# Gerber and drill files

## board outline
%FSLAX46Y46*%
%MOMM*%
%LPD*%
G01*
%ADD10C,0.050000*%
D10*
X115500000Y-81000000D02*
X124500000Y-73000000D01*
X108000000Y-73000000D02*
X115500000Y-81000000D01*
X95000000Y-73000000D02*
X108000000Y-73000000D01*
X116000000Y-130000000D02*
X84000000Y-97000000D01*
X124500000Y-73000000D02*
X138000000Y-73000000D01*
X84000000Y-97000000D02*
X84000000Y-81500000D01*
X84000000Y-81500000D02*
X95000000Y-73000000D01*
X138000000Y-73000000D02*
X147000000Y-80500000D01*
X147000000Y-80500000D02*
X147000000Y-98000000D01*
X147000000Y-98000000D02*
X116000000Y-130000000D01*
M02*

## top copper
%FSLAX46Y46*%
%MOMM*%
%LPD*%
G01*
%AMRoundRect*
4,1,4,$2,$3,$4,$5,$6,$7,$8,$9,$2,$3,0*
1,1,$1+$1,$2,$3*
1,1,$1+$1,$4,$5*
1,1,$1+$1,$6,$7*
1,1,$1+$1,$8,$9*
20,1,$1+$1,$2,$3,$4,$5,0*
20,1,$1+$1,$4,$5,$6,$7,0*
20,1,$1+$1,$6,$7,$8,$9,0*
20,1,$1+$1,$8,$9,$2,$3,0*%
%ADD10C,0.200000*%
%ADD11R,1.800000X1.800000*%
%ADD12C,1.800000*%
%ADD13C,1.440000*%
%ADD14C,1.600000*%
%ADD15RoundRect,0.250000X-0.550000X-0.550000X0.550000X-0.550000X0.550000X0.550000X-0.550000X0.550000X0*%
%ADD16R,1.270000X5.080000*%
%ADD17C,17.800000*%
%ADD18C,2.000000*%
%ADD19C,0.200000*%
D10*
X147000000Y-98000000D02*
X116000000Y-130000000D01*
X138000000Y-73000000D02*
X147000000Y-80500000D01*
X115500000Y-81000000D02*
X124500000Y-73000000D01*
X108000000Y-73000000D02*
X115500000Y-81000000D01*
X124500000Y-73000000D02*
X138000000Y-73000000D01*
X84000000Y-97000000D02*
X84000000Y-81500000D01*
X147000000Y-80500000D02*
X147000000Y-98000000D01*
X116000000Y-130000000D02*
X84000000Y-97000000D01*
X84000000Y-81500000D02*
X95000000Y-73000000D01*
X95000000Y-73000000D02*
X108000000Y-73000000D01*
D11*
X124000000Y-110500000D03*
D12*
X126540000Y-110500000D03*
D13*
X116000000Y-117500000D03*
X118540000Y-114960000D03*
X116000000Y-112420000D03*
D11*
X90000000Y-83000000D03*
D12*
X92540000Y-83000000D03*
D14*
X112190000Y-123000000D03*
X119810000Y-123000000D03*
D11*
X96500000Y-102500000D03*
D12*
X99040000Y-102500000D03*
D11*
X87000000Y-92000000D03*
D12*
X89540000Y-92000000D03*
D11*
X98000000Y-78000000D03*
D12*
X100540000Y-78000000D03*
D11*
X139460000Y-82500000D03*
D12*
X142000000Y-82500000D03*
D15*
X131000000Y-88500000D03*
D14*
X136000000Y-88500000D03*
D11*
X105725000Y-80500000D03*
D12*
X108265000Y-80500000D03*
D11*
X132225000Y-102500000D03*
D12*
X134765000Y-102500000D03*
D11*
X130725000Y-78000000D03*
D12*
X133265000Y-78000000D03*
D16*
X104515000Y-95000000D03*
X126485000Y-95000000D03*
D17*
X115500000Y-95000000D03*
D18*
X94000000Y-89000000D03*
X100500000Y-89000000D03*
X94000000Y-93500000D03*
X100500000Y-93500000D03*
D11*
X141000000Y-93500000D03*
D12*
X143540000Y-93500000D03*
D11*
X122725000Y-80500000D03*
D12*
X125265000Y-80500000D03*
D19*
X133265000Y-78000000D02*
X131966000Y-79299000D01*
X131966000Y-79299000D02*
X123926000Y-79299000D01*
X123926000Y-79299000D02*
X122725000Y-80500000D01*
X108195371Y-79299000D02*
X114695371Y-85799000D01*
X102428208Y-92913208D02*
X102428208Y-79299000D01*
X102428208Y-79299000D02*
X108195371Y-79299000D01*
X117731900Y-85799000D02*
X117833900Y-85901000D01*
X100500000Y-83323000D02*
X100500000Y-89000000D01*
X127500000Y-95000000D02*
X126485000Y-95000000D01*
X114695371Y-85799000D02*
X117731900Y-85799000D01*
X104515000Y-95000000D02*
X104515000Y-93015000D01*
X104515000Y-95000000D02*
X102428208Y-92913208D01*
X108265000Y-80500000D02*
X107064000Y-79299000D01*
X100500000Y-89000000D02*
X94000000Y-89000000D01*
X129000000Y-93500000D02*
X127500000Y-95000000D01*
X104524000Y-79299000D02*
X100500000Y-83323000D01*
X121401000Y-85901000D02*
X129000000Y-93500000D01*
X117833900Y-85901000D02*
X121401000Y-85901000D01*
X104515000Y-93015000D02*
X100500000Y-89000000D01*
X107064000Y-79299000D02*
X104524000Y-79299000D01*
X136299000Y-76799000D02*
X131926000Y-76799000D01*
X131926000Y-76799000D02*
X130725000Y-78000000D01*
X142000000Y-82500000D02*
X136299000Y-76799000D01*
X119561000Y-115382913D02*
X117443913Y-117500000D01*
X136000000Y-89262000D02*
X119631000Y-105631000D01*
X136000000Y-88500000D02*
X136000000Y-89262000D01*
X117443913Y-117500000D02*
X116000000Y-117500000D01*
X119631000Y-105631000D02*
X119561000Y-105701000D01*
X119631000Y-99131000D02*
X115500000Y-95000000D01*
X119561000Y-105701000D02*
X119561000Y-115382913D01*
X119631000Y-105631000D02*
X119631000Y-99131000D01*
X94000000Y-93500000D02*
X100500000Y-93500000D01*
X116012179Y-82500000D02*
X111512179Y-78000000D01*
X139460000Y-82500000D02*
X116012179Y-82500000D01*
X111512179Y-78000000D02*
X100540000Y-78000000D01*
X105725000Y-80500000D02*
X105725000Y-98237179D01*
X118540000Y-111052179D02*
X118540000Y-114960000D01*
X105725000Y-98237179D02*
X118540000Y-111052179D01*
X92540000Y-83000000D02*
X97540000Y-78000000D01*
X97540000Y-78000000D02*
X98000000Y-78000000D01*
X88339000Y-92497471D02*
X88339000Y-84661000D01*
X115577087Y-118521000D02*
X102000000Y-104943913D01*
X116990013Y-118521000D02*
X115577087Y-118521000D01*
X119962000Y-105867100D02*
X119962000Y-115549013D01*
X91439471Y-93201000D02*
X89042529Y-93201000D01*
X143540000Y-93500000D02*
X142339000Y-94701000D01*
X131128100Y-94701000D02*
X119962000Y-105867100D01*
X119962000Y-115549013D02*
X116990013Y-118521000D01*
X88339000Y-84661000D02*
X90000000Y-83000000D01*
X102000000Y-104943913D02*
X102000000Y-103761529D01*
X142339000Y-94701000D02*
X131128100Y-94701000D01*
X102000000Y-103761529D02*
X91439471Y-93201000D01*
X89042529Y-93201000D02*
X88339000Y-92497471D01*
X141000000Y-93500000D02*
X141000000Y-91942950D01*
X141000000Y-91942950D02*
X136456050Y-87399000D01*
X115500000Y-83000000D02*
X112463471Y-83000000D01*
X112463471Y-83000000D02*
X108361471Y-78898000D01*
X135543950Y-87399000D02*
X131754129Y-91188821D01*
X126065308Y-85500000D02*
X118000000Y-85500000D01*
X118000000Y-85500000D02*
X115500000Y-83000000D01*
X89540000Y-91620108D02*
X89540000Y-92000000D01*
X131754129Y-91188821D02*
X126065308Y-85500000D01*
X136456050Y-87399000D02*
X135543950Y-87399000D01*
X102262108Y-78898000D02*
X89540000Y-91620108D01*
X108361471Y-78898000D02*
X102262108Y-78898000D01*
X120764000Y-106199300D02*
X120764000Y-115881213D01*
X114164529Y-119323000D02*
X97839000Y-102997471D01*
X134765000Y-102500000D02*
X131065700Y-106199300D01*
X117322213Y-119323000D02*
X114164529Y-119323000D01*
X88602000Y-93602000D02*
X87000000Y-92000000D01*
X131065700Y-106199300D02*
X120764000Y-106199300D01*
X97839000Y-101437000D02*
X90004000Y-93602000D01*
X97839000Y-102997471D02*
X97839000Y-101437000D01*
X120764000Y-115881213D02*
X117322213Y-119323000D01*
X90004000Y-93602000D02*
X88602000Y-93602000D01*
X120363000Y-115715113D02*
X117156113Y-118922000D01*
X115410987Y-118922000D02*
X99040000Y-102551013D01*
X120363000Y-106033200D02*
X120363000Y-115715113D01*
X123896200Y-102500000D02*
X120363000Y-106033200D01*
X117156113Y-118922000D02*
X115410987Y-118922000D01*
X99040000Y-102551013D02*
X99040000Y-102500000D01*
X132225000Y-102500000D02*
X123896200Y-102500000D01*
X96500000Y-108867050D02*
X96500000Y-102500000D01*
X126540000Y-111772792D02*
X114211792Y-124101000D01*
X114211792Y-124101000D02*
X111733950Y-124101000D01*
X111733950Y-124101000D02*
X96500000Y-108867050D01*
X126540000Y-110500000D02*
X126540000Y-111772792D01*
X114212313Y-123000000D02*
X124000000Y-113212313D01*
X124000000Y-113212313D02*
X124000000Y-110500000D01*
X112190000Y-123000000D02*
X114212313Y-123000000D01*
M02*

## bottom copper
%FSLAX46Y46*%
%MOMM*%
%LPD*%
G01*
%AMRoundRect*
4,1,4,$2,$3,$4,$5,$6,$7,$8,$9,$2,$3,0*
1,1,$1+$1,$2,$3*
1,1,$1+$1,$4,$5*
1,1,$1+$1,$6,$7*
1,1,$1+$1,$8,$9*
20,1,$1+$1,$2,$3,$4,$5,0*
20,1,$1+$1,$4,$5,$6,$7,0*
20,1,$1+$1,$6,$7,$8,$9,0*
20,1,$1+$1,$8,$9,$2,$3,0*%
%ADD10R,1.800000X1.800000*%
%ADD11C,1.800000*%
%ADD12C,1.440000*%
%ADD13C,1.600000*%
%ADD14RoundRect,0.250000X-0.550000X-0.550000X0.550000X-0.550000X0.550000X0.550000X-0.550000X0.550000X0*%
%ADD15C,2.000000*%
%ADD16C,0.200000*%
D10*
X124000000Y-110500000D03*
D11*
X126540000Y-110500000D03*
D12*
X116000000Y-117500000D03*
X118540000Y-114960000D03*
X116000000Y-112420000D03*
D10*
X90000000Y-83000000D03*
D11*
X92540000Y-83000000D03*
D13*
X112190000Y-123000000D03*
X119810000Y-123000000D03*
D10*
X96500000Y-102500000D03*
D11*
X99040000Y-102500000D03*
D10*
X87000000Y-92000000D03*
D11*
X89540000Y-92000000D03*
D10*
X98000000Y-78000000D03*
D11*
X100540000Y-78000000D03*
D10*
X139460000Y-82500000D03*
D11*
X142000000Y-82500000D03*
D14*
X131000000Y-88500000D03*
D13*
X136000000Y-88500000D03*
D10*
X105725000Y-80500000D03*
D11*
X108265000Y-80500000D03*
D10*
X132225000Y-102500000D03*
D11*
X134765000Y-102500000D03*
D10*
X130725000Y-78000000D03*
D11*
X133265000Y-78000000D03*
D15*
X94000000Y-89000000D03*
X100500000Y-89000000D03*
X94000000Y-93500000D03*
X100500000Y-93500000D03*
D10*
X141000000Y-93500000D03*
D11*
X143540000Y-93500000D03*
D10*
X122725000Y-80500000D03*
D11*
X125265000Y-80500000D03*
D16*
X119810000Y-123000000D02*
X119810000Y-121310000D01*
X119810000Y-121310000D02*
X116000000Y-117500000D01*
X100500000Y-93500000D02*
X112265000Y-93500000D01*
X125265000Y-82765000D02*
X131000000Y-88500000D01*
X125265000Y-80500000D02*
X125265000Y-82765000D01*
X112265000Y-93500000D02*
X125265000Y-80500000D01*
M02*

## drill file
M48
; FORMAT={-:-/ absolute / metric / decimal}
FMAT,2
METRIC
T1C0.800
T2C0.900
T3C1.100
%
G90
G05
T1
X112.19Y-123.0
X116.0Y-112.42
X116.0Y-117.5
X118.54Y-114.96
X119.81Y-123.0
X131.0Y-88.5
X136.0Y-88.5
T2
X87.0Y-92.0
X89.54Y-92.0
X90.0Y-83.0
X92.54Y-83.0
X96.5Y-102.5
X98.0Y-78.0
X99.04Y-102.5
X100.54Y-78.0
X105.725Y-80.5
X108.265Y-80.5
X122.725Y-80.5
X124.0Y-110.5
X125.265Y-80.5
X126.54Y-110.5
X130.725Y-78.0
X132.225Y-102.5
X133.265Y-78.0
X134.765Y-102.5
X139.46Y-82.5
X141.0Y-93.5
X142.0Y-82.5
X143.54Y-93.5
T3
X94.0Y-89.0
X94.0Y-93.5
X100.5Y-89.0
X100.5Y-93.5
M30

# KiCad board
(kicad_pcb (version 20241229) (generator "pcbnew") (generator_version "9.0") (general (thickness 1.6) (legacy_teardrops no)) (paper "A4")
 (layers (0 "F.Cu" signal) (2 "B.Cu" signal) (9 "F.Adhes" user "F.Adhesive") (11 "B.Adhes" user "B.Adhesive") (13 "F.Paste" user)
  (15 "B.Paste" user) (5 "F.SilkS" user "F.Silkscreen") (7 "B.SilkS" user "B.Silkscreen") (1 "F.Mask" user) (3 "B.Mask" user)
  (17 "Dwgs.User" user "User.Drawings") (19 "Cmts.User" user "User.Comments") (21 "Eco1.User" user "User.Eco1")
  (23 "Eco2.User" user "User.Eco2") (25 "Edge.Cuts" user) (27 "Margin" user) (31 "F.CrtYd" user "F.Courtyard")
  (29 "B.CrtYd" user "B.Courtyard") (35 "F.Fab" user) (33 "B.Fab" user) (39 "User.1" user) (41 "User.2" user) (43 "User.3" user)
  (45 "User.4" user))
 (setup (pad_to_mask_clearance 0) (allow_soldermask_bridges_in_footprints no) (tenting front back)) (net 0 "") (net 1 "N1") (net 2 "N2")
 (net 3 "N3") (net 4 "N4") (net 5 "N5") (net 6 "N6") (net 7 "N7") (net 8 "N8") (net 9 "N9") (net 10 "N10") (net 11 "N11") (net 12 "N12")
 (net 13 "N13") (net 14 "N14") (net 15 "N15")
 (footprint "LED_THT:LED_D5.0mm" (layer "F.Cu") (at 124 110.5)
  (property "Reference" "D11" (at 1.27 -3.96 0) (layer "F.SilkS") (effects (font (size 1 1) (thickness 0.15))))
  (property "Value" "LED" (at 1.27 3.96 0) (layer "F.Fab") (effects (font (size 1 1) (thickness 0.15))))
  (pad "1" thru_hole rect (at 0 0) (size 1.8 1.8) (drill 0.9) (layers "*.Cu" "*.Mask") (remove_unused_layers no) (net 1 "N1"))
  (pad "2" thru_hole circle (at 2.54 0) (size 1.8 1.8) (drill 0.9) (layers "*.Cu" "*.Mask") (remove_unused_layers no) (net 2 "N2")))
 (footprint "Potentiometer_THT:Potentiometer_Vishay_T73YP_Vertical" (layer "F.Cu") (at 116 117.5)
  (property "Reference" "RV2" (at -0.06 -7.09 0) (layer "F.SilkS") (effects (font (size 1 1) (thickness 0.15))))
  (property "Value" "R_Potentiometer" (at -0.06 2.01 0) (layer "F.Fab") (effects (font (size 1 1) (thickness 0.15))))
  (pad "1" thru_hole circle (at 0 0) (size 1.44 1.44) (drill 0.8) (layers "*.Cu" "*.Mask") (remove_unused_layers no) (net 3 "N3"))
  (pad "2" thru_hole circle (at 2.54 -2.54) (size 1.44 1.44) (drill 0.8) (layers "*.Cu" "*.Mask") (remove_unused_layers no) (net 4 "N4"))
  (pad "3" thru_hole circle (at 0 -5.08) (size 1.44 1.44) (drill 0.8) (layers "*.Cu" "*.Mask") (remove_unused_layers no) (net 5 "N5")))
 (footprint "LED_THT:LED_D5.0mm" (layer "F.Cu") (at 90 83)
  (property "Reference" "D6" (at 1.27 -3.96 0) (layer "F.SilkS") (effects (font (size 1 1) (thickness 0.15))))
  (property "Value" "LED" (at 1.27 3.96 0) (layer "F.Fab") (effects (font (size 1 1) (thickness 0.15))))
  (pad "1" thru_hole rect (at 0 0) (size 1.8 1.8) (drill 0.9) (layers "*.Cu" "*.Mask") (remove_unused_layers no) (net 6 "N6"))
  (pad "2" thru_hole circle (at 2.54 0) (size 1.8 1.8) (drill 0.9) (layers "*.Cu" "*.Mask") (remove_unused_layers no) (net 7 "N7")))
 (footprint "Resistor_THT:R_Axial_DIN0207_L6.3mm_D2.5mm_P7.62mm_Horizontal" (layer "F.Cu") (at 112.19 123)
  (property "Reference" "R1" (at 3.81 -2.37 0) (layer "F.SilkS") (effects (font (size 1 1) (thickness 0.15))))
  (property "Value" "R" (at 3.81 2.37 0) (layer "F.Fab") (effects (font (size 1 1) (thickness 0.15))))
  (pad "1" thru_hole circle (at 0 0) (size 1.6 1.6) (drill 0.8) (layers "*.Cu" "*.Mask") (remove_unused_layers no) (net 1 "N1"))
  (pad "2" thru_hole circle (at 7.62 0) (size 1.6 1.6) (drill 0.8) (layers "*.Cu" "*.Mask") (remove_unused_layers no) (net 3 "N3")))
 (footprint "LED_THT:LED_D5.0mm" (layer "F.Cu") (at 96.5 102.5)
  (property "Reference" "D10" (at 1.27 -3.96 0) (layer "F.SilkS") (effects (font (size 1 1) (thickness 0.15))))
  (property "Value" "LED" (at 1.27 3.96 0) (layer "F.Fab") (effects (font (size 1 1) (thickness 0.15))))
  (pad "1" thru_hole rect (at 0 0) (size 1.8 1.8) (drill 0.9) (layers "*.Cu" "*.Mask") (remove_unused_layers no) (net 2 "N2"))
  (pad "2" thru_hole circle (at 2.54 0) (size 1.8 1.8) (drill 0.9) (layers "*.Cu" "*.Mask") (remove_unused_layers no) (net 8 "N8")))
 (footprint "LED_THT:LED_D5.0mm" (layer "F.Cu") (at 87 92)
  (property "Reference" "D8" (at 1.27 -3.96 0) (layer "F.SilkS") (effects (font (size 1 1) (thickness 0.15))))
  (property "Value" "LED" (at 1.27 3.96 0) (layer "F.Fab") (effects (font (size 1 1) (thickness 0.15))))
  (pad "1" thru_hole rect (at 0 0) (size 1.8 1.8) (drill 0.9) (layers "*.Cu" "*.Mask") (remove_unused_layers no) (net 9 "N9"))
  (pad "2" thru_hole circle (at 2.54 0) (size 1.8 1.8) (drill 0.9) (layers "*.Cu" "*.Mask") (remove_unused_layers no) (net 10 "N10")))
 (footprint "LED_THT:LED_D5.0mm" (layer "F.Cu") (at 98 78)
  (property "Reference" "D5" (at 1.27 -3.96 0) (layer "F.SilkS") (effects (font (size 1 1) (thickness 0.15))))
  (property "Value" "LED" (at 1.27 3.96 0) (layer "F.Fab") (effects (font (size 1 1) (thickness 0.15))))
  (pad "1" thru_hole rect (at 0 0) (size 1.8 1.8) (drill 0.9) (layers "*.Cu" "*.Mask") (remove_unused_layers no) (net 7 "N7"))
  (pad "2" thru_hole circle (at 2.54 0) (size 1.8 1.8) (drill 0.9) (layers "*.Cu" "*.Mask") (remove_unused_layers no) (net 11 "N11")))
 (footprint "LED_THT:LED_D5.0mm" (layer "F.Cu") (at 139.46 82.5)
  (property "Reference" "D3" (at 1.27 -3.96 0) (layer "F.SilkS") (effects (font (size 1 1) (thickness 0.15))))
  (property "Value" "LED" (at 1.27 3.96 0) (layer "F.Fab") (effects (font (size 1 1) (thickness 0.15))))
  (pad "1" thru_hole rect (at 0 0) (size 1.8 1.8) (drill 0.9) (layers "*.Cu" "*.Mask") (remove_unused_layers no) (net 11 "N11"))
  (pad "2" thru_hole circle (at 2.54 0) (size 1.8 1.8) (drill 0.9) (layers "*.Cu" "*.Mask") (remove_unused_layers no) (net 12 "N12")))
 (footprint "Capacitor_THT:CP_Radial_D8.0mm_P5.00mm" (layer "F.Cu") (at 131 88.5)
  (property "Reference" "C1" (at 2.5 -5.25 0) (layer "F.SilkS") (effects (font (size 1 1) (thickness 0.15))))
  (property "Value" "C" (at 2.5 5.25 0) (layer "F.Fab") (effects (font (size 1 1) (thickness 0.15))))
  (pad "1" thru_hole roundrect (at 0 0) (size 1.6 1.6) (drill 0.8) (layers "*.Cu" "*.Mask") (remove_unused_layers no)
   (roundrect_rratio 0.15625) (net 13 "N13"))
  (pad "2" thru_hole circle (at 5 0) (size 1.6 1.6) (drill 0.8) (layers "*.Cu" "*.Mask") (remove_unused_layers no) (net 3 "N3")))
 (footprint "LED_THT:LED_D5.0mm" (layer "F.Cu") (at 105.725 80.5)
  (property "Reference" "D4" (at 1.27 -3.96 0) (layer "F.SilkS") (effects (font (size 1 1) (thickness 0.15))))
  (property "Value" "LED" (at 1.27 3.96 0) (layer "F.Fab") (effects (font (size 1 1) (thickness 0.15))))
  (pad "1" thru_hole rect (at 0 0) (size 1.8 1.8) (drill 0.9) (layers "*.Cu" "*.Mask") (remove_unused_layers no) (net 4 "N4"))
  (pad "2" thru_hole circle (at 2.54 0) (size 1.8 1.8) (drill 0.9) (layers "*.Cu" "*.Mask") (remove_unused_layers no) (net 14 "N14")))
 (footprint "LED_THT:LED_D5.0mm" (layer "F.Cu") (at 132.225 102.5)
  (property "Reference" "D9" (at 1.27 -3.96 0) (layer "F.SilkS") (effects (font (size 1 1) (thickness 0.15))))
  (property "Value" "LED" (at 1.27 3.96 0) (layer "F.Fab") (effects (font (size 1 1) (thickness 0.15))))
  (pad "1" thru_hole rect (at 0 0) (size 1.8 1.8) (drill 0.9) (layers "*.Cu" "*.Mask") (remove_unused_layers no) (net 8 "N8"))
  (pad "2" thru_hole circle (at 2.54 0) (size 1.8 1.8) (drill 0.9) (layers "*.Cu" "*.Mask") (remove_unused_layers no) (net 9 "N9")))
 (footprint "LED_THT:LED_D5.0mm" (layer "F.Cu") (at 130.725 78)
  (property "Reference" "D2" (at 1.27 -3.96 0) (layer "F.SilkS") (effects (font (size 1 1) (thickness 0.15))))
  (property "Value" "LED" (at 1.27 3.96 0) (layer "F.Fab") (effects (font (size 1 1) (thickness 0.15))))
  (pad "1" thru_hole rect (at 0 0) (size 1.8 1.8) (drill 0.9) (layers "*.Cu" "*.Mask") (remove_unused_layers no) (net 12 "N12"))
  (pad "2" thru_hole circle (at 2.54 0) (size 1.8 1.8) (drill 0.9) (layers "*.Cu" "*.Mask") (remove_unused_layers no) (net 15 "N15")))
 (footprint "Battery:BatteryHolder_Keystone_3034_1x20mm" (layer "F.Cu") (at 115.5 95)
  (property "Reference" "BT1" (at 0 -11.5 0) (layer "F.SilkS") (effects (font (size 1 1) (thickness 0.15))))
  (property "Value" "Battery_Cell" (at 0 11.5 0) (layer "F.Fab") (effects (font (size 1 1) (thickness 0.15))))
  (pad "1" smd rect (at -10.985 0) (size 1.27 5.08) (layers "F.Cu" "F.Mask" "F.Paste") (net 14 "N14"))
  (pad "1" smd rect (at 10.985 0) (size 1.27 5.08) (layers "F.Cu" "F.Mask" "F.Paste") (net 14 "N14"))
  (pad "2" smd circle (at 0 0) (size 17.8 17.8) (layers "F.Cu" "F.Mask") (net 3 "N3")))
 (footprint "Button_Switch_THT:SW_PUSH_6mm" (layer "F.Cu") (at 94 89)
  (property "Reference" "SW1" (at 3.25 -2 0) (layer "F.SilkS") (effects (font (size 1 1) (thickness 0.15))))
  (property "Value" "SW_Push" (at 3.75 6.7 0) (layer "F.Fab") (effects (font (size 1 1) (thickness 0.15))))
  (pad "1" thru_hole circle (at 0 0 90) (size 2 2) (drill 1.1) (layers "*.Cu" "*.Mask") (remove_unused_layers no) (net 14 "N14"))
  (pad "1" thru_hole circle (at 6.5 0 90) (size 2 2) (drill 1.1) (layers "*.Cu" "*.Mask") (remove_unused_layers no) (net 14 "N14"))
  (pad "2" thru_hole circle (at 0 4.5 90) (size 2 2) (drill 1.1) (layers "*.Cu" "*.Mask") (remove_unused_layers no) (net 13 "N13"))
  (pad "2" thru_hole circle (at 6.5 4.5 90) (size 2 2) (drill 1.1) (layers "*.Cu" "*.Mask") (remove_unused_layers no) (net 13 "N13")))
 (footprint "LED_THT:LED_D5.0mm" (layer "F.Cu") (at 141 93.5)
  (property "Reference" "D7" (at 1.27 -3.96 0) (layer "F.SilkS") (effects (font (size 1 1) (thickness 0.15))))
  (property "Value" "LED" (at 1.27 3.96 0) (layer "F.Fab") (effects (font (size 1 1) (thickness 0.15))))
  (pad "1" thru_hole rect (at 0 0) (size 1.8 1.8) (drill 0.9) (layers "*.Cu" "*.Mask") (remove_unused_layers no) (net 10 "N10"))
  (pad "2" thru_hole circle (at 2.54 0) (size 1.8 1.8) (drill 0.9) (layers "*.Cu" "*.Mask") (remove_unused_layers no) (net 6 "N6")))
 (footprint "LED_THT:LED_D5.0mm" (layer "F.Cu") (at 122.725 80.5)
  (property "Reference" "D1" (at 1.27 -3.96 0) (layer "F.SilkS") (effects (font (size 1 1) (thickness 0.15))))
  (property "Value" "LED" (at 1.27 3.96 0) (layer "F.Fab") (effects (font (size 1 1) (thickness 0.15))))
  (pad "1" thru_hole rect (at 0 0) (size 1.8 1.8) (drill 0.9) (layers "*.Cu" "*.Mask") (remove_unused_layers no) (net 15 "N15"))
  (pad "2" thru_hole circle (at 2.54 0) (size 1.8 1.8) (drill 0.9) (layers "*.Cu" "*.Mask") (remove_unused_layers no) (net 13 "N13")))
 (gr_line (start 147 98) (end 116 130) (stroke (width 0.2) (type default)) (layer "F.Cu"))
 (gr_line (start 138 73) (end 147 80.5) (stroke (width 0.2) (type default)) (layer "F.Cu"))
 (gr_line (start 115.5 81) (end 124.5 73) (stroke (width 0.2) (type default)) (layer "F.Cu"))
 (gr_line (start 108 73) (end 115.5 81) (stroke (width 0.2) (type default)) (layer "F.Cu"))
 (gr_line (start 124.5 73) (end 138 73) (stroke (width 0.2) (type default)) (layer "F.Cu"))
 (gr_line (start 84 97) (end 84 81.5) (stroke (width 0.2) (type default)) (layer "F.Cu"))
 (gr_line (start 147 80.5) (end 147 98) (stroke (width 0.2) (type default)) (layer "F.Cu"))
 (gr_line (start 116 130) (end 84 97) (stroke (width 0.2) (type default)) (layer "F.Cu"))
 (gr_line (start 84 81.5) (end 95 73) (stroke (width 0.2) (type default)) (layer "F.Cu"))
 (gr_line (start 95 73) (end 108 73) (stroke (width 0.2) (type default)) (layer "F.Cu"))
 (gr_line (start 115.5 81) (end 124.5 73) (stroke (width 0.05) (type default)) (layer "Edge.Cuts"))
 (gr_line (start 108 73) (end 115.5 81) (stroke (width 0.05) (type default)) (layer "Edge.Cuts"))
 (gr_line (start 95 73) (end 108 73) (stroke (width 0.05) (type default)) (layer "Edge.Cuts"))
 (gr_line (start 116 130) (end 84 97) (stroke (width 0.05) (type default)) (layer "Edge.Cuts"))
 (gr_line (start 124.5 73) (end 138 73) (stroke (width 0.05) (type default)) (layer "Edge.Cuts"))
 (gr_line (start 84 97) (end 84 81.5) (stroke (width 0.05) (type default)) (layer "Edge.Cuts"))
 (gr_line (start 84 81.5) (end 95 73) (stroke (width 0.05) (type default)) (layer "Edge.Cuts"))
 (gr_line (start 138 73) (end 147 80.5) (stroke (width 0.05) (type default)) (layer "Edge.Cuts"))
 (gr_line (start 147 80.5) (end 147 98) (stroke (width 0.05) (type default)) (layer "Edge.Cuts"))
 (gr_line (start 147 98) (end 116 130) (stroke (width 0.05) (type default)) (layer "Edge.Cuts"))
 (segment (start 133.265 78) (end 131.966 79.299) (width 0.2) (layer "F.Cu") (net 15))
 (segment (start 131.966 79.299) (end 123.926 79.299) (width 0.2) (layer "F.Cu") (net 15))
 (segment (start 123.926 79.299) (end 122.725 80.5) (width 0.2) (layer "F.Cu") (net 15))
 (segment (start 108.195371 79.299) (end 114.695371 85.799) (width 0.2) (layer "F.Cu") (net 14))
 (segment (start 102.428208 92.913208) (end 102.428208 79.299) (width 0.2) (layer "F.Cu") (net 14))
 (segment (start 102.428208 79.299) (end 108.195371 79.299) (width 0.2) (layer "F.Cu") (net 14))
 (segment (start 117.7319 85.799) (end 117.8339 85.901) (width 0.2) (layer "F.Cu") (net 14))
 (segment (start 100.5 83.323) (end 100.5 89) (width 0.2) (layer "F.Cu") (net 14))
 (segment (start 127.5 95) (end 126.485 95) (width 0.2) (layer "F.Cu") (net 14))
 (segment (start 114.695371 85.799) (end 117.7319 85.799) (width 0.2) (layer "F.Cu") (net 14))
 (segment (start 104.515 95) (end 104.515 93.015) (width 0.2) (layer "F.Cu") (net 14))
 (segment (start 104.515 95) (end 102.428208 92.913208) (width 0.2) (layer "F.Cu") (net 14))
 (segment (start 108.265 80.5) (end 107.064 79.299) (width 0.2) (layer "F.Cu") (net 14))
 (segment (start 100.5 89) (end 94 89) (width 0.2) (layer "F.Cu") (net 14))
 (segment (start 129 93.5) (end 127.5 95) (width 0.2) (layer "F.Cu") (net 14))
 (segment (start 104.524 79.299) (end 100.5 83.323) (width 0.2) (layer "F.Cu") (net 14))
 (segment (start 121.401 85.901) (end 129 93.5) (width 0.2) (layer "F.Cu") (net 14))
 (segment (start 117.8339 85.901) (end 121.401 85.901) (width 0.2) (layer "F.Cu") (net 14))
 (segment (start 104.515 93.015) (end 100.5 89) (width 0.2) (layer "F.Cu") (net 14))
 (segment (start 107.064 79.299) (end 104.524 79.299) (width 0.2) (layer "F.Cu") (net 14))
 (segment (start 136.299 76.799) (end 131.926 76.799) (width 0.2) (layer "F.Cu") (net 12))
 (segment (start 131.926 76.799) (end 130.725 78) (width 0.2) (layer "F.Cu") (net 12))
 (segment (start 142 82.5) (end 136.299 76.799) (width 0.2) (layer "F.Cu") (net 12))
 (segment (start 119.561 115.382913) (end 117.443913 117.5) (width 0.2) (layer "F.Cu") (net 3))
 (segment (start 136 89.262) (end 119.631 105.631) (width 0.2) (layer "F.Cu") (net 3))
 (segment (start 136 88.5) (end 136 89.262) (width 0.2) (layer "F.Cu") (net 3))
 (segment (start 117.443913 117.5) (end 116 117.5) (width 0.2) (layer "F.Cu") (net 3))
 (segment (start 119.631 105.631) (end 119.561 105.701) (width 0.2) (layer "F.Cu") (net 3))
 (segment (start 119.631 99.131) (end 115.5 95) (width 0.2) (layer "F.Cu") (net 3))
 (segment (start 119.561 105.701) (end 119.561 115.382913) (width 0.2) (layer "F.Cu") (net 3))
 (segment (start 119.631 105.631) (end 119.631 99.131) (width 0.2) (layer "F.Cu") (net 3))
 (segment (start 119.81 123) (end 119.81 121.31) (width 0.2) (layer "B.Cu") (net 3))
 (segment (start 119.81 121.31) (end 116 117.5) (width 0.2) (layer "B.Cu") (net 3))
 (segment (start 94 93.5) (end 100.5 93.5) (width 0.2) (layer "F.Cu") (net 13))
 (segment (start 100.5 93.5) (end 112.265 93.5) (width 0.2) (layer "B.Cu") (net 13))
 (segment (start 125.265 82.765) (end 131 88.5) (width 0.2) (layer "B.Cu") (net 13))
 (segment (start 125.265 80.5) (end 125.265 82.765) (width 0.2) (layer "B.Cu") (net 13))
 (segment (start 112.265 93.5) (end 125.265 80.5) (width 0.2) (layer "B.Cu") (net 13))
 (segment (start 116.012179 82.5) (end 111.512179 78) (width 0.2) (layer "F.Cu") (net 11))
 (segment (start 139.46 82.5) (end 116.012179 82.5) (width 0.2) (layer "F.Cu") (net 11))
 (segment (start 111.512179 78) (end 100.54 78) (width 0.2) (layer "F.Cu") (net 11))
 (segment (start 105.725 80.5) (end 105.725 98.237179) (width 0.2) (layer "F.Cu") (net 4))
 (segment (start 118.54 111.052179) (end 118.54 114.96) (width 0.2) (layer "F.Cu") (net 4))
 (segment (start 105.725 98.237179) (end 118.54 111.052179) (width 0.2) (layer "F.Cu") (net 4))
 (segment (start 92.54 83) (end 97.54 78) (width 0.2) (layer "F.Cu") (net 7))
 (segment (start 97.54 78) (end 98 78) (width 0.2) (layer "F.Cu") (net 7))
 (segment (start 88.339 92.497471) (end 88.339 84.661) (width 0.2) (layer "F.Cu") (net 6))
 (segment (start 115.577087 118.521) (end 102 104.943913) (width 0.2) (layer "F.Cu") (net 6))
 (segment (start 116.990013 118.521) (end 115.577087 118.521) (width 0.2) (layer "F.Cu") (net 6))
 (segment (start 119.962 105.8671) (end 119.962 115.549013) (width 0.2) (layer "F.Cu") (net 6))
 (segment (start 91.439471 93.201) (end 89.042529 93.201) (width 0.2) (layer "F.Cu") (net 6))
 (segment (start 143.54 93.5) (end 142.339 94.701) (width 0.2) (layer "F.Cu") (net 6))
 (segment (start 131.1281 94.701) (end 119.962 105.8671) (width 0.2) (layer "F.Cu") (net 6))
 (segment (start 119.962 115.549013) (end 116.990013 118.521) (width 0.2) (layer "F.Cu") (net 6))
 (segment (start 88.339 84.661) (end 90 83) (width 0.2) (layer "F.Cu") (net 6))
 (segment (start 102 104.943913) (end 102 103.761529) (width 0.2) (layer "F.Cu") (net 6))
 (segment (start 142.339 94.701) (end 131.1281 94.701) (width 0.2) (layer "F.Cu") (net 6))
 (segment (start 102 103.761529) (end 91.439471 93.201) (width 0.2) (layer "F.Cu") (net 6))
 (segment (start 89.042529 93.201) (end 88.339 92.497471) (width 0.2) (layer "F.Cu") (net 6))
 (segment (start 141 93.5) (end 141 91.94295) (width 0.2) (layer "F.Cu") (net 10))
 (segment (start 141 91.94295) (end 136.45605 87.399) (width 0.2) (layer "F.Cu") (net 10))
 (segment (start 115.5 83) (end 112.463471 83) (width 0.2) (layer "F.Cu") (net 10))
 (segment (start 112.463471 83) (end 108.361471 78.898) (width 0.2) (layer "F.Cu") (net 10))
 (segment (start 135.54395 87.399) (end 131.754129 91.188821) (width 0.2) (layer "F.Cu") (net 10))
 (segment (start 126.065308 85.5) (end 118 85.5) (width 0.2) (layer "F.Cu") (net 10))
 (segment (start 118 85.5) (end 115.5 83) (width 0.2) (layer "F.Cu") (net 10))
 (segment (start 89.54 91.620108) (end 89.54 92) (width 0.2) (layer "F.Cu") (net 10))
 (segment (start 131.754129 91.188821) (end 126.065308 85.5) (width 0.2) (layer "F.Cu") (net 10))
 (segment (start 136.45605 87.399) (end 135.54395 87.399) (width 0.2) (layer "F.Cu") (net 10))
 (segment (start 102.262108 78.898) (end 89.54 91.620108) (width 0.2) (layer "F.Cu") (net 10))
 (segment (start 108.361471 78.898) (end 102.262108 78.898) (width 0.2) (layer "F.Cu") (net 10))
 (segment (start 120.764 106.1993) (end 120.764 115.881213) (width 0.2) (layer "F.Cu") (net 9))
 (segment (start 114.164529 119.323) (end 97.839 102.997471) (width 0.2) (layer "F.Cu") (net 9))
 (segment (start 134.765 102.5) (end 131.0657 106.1993) (width 0.2) (layer "F.Cu") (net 9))
 (segment (start 117.322213 119.323) (end 114.164529 119.323) (width 0.2) (layer "F.Cu") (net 9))
 (segment (start 88.602 93.602) (end 87 92) (width 0.2) (layer "F.Cu") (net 9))
 (segment (start 131.0657 106.1993) (end 120.764 106.1993) (width 0.2) (layer "F.Cu") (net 9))
 (segment (start 97.839 101.437) (end 90.004 93.602) (width 0.2) (layer "F.Cu") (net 9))
 (segment (start 97.839 102.997471) (end 97.839 101.437) (width 0.2) (layer "F.Cu") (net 9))
 (segment (start 120.764 115.881213) (end 117.322213 119.323) (width 0.2) (layer "F.Cu") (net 9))
 (segment (start 90.004 93.602) (end 88.602 93.602) (width 0.2) (layer "F.Cu") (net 9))
 (segment (start 120.363 115.715113) (end 117.156113 118.922) (width 0.2) (layer "F.Cu") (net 8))
 (segment (start 115.410987 118.922) (end 99.04 102.551013) (width 0.2) (layer "F.Cu") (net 8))
 (segment (start 120.363 106.0332) (end 120.363 115.715113) (width 0.2) (layer "F.Cu") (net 8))
 (segment (start 123.8962 102.5) (end 120.363 106.0332) (width 0.2) (layer "F.Cu") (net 8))
 (segment (start 117.156113 118.922) (end 115.410987 118.922) (width 0.2) (layer "F.Cu") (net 8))
 (segment (start 99.04 102.551013) (end 99.04 102.5) (width 0.2) (layer "F.Cu") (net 8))
 (segment (start 132.225 102.5) (end 123.8962 102.5) (width 0.2) (layer "F.Cu") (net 8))
 (segment (start 96.5 108.86705) (end 96.5 102.5) (width 0.2) (layer "F.Cu") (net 2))
 (segment (start 126.54 111.772792) (end 114.211792 124.101) (width 0.2) (layer "F.Cu") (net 2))
 (segment (start 114.211792 124.101) (end 111.73395 124.101) (width 0.2) (layer "F.Cu") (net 2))
 (segment (start 111.73395 124.101) (end 96.5 108.86705) (width 0.2) (layer "F.Cu") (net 2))
 (segment (start 126.54 110.5) (end 126.54 111.772792) (width 0.2) (layer "F.Cu") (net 2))
 (segment (start 114.212313 123) (end 124 113.212313) (width 0.2) (layer "F.Cu") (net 1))
 (segment (start 124 113.212313) (end 124 110.5) (width 0.2) (layer "F.Cu") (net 1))
 (segment (start 112.19 123) (end 114.212313 123) (width 0.2) (layer "F.Cu") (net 1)))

